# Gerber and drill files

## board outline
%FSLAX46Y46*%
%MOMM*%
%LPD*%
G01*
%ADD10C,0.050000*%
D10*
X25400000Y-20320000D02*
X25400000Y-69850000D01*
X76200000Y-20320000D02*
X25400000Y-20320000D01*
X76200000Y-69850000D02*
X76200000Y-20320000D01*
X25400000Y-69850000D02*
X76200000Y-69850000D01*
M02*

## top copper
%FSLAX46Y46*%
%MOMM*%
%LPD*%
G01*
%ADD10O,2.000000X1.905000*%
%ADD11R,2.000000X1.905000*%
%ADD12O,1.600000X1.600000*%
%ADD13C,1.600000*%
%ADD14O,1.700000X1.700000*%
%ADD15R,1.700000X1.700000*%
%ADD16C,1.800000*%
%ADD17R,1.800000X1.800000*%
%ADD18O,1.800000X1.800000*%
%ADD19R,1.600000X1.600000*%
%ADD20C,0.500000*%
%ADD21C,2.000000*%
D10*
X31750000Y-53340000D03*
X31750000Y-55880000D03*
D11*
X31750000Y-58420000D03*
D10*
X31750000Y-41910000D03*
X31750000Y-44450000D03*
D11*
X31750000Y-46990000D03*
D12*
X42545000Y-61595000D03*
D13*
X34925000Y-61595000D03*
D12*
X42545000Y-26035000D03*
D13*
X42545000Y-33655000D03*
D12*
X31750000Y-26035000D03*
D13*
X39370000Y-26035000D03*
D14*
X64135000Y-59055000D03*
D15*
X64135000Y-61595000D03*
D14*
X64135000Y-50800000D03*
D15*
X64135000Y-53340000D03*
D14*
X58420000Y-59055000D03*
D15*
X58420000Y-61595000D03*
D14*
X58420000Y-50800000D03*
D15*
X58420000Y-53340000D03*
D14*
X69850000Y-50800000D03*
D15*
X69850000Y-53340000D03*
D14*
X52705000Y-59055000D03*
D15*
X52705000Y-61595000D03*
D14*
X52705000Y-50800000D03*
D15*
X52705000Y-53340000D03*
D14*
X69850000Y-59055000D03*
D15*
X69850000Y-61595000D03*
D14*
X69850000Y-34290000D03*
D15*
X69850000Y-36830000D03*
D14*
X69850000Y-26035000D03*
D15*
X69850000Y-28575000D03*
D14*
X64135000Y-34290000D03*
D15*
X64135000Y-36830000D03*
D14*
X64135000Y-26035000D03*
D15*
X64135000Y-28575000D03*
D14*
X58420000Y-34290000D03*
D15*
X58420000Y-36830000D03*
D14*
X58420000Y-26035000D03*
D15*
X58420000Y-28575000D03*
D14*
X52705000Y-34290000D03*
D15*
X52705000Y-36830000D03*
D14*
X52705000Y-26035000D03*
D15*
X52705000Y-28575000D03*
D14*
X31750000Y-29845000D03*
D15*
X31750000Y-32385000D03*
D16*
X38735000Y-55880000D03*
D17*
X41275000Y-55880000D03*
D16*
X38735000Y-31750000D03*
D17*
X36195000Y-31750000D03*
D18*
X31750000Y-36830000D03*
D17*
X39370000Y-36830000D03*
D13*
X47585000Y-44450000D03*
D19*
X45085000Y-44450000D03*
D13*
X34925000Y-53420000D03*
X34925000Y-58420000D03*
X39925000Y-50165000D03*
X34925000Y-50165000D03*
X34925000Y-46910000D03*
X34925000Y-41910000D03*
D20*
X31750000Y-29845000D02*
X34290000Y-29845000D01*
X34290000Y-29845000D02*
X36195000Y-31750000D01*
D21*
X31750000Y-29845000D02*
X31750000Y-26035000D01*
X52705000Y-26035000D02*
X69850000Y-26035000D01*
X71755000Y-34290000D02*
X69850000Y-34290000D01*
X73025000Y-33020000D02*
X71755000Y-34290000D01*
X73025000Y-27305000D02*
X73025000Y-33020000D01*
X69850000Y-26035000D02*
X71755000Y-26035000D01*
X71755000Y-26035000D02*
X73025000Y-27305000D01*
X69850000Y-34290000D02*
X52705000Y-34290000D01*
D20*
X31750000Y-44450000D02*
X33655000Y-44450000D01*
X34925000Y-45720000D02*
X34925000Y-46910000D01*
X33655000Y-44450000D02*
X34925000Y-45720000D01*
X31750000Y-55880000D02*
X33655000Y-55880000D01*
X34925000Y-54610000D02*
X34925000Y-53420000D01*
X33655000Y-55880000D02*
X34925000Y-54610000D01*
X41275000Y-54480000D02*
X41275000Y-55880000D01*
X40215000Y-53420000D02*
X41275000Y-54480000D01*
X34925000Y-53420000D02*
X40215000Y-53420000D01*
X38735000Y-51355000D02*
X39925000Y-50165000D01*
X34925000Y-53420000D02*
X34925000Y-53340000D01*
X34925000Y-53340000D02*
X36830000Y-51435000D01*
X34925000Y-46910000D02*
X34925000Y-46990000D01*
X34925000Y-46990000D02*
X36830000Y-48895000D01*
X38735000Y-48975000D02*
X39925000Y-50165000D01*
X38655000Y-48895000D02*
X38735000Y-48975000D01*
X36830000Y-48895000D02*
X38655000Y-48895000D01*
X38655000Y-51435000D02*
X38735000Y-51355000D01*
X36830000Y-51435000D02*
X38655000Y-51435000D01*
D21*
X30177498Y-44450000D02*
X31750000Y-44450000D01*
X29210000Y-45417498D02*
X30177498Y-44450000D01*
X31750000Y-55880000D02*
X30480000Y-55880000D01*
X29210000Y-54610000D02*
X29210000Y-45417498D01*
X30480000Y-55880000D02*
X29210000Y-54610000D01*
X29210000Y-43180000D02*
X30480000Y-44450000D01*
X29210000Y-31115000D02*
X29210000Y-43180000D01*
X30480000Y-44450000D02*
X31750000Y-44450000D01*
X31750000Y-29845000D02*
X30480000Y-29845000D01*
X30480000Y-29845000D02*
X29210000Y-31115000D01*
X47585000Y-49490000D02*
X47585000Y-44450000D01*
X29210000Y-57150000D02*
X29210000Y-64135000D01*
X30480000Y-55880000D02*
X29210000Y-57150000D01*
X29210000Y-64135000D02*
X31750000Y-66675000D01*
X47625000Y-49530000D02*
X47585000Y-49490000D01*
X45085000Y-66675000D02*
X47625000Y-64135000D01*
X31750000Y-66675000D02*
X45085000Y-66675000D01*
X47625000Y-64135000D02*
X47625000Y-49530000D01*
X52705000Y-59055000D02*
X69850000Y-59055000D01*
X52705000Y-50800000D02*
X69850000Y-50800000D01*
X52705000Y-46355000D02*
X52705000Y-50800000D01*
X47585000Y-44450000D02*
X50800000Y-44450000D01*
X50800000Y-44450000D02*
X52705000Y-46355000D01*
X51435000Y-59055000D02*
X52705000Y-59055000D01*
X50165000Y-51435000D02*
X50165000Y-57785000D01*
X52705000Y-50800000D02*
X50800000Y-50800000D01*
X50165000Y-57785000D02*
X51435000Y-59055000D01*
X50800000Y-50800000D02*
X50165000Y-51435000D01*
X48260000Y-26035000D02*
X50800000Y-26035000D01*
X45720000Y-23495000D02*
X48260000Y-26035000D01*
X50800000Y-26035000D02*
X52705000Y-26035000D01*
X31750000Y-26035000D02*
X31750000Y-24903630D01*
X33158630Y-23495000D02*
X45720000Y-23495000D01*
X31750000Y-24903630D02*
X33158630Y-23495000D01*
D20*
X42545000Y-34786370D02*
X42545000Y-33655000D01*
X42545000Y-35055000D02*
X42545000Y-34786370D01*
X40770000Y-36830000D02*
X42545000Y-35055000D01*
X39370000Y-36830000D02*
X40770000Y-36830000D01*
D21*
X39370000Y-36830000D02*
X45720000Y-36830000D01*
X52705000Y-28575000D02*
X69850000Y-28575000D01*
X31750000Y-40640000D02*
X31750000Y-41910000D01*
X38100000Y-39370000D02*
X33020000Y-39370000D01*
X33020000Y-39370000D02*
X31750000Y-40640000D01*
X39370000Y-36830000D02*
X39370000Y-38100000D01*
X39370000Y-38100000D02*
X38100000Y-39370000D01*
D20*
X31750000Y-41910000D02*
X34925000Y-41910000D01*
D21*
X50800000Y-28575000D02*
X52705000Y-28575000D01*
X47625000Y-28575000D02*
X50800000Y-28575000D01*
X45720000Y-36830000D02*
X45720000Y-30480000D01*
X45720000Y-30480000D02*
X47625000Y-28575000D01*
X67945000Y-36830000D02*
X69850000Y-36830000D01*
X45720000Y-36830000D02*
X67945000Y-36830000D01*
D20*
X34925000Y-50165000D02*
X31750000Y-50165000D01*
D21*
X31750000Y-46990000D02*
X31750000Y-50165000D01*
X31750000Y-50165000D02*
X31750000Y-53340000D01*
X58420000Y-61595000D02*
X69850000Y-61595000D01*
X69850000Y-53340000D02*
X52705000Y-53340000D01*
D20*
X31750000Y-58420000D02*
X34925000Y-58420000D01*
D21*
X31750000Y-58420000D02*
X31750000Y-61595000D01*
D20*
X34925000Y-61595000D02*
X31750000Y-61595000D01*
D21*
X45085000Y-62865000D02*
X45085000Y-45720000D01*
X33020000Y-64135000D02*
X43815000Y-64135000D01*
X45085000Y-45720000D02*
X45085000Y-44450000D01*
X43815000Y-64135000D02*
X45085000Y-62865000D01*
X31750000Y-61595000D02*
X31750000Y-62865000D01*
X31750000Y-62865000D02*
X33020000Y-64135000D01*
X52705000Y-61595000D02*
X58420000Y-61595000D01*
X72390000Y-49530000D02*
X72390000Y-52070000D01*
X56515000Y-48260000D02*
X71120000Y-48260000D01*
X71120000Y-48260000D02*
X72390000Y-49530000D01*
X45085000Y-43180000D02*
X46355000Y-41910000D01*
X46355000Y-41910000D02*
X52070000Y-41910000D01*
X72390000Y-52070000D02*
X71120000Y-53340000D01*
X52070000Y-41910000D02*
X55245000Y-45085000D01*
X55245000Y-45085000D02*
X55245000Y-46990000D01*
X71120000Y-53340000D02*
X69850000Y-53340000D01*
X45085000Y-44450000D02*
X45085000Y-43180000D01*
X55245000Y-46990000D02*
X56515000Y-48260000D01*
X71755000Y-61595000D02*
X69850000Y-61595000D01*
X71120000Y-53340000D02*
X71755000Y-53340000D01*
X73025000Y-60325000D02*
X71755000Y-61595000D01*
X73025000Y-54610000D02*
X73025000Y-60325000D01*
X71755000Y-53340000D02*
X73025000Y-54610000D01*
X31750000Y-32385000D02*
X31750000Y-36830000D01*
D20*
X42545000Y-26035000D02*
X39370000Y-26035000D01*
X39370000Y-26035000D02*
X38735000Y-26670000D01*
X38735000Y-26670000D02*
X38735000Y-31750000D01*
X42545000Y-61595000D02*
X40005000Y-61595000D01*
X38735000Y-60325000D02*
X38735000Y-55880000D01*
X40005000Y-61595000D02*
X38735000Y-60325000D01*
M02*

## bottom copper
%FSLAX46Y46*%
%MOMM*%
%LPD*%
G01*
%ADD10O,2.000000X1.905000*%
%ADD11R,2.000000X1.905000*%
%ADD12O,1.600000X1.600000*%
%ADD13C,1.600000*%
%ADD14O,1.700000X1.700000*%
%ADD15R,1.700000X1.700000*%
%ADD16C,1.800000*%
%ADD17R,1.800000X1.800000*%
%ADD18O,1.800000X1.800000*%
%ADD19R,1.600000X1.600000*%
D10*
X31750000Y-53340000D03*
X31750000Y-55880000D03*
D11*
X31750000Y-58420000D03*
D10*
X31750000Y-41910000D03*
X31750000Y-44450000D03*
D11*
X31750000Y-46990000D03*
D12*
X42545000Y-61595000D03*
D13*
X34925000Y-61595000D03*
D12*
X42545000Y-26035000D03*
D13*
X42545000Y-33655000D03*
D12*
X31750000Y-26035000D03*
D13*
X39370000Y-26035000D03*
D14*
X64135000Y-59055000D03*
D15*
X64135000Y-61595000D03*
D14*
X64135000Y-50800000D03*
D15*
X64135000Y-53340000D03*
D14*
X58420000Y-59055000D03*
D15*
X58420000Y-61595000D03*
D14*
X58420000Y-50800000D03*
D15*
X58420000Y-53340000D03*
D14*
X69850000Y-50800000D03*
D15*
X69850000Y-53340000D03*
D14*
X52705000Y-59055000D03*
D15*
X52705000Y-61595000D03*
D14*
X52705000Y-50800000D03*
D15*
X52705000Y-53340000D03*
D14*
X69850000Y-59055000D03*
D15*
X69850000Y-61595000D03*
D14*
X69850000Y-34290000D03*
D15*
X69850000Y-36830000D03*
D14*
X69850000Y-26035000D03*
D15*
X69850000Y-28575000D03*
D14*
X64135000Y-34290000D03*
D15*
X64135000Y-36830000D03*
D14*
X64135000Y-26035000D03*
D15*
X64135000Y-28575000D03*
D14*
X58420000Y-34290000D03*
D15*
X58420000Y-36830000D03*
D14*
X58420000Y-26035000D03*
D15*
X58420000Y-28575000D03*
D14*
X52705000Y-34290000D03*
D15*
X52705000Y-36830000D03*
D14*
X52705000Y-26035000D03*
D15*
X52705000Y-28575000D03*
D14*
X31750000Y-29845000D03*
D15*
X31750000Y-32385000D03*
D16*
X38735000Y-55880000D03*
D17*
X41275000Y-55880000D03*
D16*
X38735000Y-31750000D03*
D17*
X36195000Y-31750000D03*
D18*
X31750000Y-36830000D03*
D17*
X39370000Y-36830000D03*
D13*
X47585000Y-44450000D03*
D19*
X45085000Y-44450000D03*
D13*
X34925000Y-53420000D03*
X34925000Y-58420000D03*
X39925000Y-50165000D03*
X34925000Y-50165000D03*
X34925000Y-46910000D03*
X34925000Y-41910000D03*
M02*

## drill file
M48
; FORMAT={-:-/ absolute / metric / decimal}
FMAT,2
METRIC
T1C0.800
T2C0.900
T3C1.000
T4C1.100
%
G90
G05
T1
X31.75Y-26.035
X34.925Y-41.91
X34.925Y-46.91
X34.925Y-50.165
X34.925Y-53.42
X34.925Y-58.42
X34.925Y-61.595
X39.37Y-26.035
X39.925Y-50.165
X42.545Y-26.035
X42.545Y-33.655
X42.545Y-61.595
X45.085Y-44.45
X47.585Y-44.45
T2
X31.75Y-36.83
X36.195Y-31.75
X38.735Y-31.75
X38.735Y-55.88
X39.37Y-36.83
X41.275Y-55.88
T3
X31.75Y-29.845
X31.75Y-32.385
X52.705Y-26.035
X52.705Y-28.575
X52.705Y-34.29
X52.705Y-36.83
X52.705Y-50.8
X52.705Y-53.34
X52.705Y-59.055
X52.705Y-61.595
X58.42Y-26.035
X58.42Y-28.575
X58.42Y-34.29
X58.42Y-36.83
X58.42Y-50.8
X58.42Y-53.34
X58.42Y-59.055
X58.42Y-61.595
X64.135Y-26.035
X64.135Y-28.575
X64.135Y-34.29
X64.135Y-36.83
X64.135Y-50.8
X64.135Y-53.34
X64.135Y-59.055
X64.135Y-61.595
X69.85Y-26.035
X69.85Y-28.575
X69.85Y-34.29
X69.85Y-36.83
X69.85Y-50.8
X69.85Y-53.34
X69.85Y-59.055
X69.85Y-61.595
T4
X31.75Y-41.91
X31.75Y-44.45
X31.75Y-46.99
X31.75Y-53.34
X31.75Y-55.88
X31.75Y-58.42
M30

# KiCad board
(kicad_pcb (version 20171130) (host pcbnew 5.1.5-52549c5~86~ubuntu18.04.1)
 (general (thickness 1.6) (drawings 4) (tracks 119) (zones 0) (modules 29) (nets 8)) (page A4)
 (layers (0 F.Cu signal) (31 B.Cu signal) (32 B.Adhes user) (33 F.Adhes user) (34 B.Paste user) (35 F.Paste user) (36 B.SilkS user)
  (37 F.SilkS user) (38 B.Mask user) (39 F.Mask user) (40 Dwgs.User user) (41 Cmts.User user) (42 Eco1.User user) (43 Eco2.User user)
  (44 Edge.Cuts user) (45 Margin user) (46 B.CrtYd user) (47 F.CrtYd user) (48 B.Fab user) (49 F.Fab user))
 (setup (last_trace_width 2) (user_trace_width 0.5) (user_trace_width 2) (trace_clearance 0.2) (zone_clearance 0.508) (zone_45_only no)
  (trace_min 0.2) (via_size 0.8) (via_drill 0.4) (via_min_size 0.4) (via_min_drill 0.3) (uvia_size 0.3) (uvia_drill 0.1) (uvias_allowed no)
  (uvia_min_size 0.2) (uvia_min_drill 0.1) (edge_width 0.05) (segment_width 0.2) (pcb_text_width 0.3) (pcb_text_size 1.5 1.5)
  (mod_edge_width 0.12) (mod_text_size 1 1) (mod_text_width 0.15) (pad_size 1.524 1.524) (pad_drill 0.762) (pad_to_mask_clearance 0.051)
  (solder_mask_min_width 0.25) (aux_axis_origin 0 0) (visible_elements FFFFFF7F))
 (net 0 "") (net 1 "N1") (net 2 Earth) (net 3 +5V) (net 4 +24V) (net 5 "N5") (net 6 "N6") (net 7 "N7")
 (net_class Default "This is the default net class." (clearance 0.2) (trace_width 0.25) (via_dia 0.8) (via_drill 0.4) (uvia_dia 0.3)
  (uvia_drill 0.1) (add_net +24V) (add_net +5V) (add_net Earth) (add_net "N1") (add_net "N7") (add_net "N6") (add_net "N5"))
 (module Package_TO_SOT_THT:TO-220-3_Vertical (layer F.Cu) (at 31.75 58.42 90)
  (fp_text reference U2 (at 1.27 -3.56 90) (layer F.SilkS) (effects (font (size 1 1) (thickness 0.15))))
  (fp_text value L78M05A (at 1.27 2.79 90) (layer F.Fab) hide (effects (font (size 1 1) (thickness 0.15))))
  (pad 3 thru_hole oval (at 5.08 0 90) (size 1.905 2) (drill 1.1) (layers *.Cu *.Mask) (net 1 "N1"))
  (pad 2 thru_hole oval (at 2.54 0 90) (size 1.905 2) (drill 1.1) (layers *.Cu *.Mask) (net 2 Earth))
  (pad 1 thru_hole rect (at 0 0 90) (size 1.905 2) (drill 1.1) (layers *.Cu *.Mask) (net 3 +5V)))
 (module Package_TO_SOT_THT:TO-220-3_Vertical (layer F.Cu) (at 31.75 46.99 90)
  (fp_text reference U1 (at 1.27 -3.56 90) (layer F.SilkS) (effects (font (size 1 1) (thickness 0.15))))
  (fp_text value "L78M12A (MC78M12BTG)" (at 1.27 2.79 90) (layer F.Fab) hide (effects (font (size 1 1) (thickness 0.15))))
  (pad 3 thru_hole oval (at 5.08 0 90) (size 1.905 2) (drill 1.1) (layers *.Cu *.Mask) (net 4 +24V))
  (pad 2 thru_hole oval (at 2.54 0 90) (size 1.905 2) (drill 1.1) (layers *.Cu *.Mask) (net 2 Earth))
  (pad 1 thru_hole rect (at 0 0 90) (size 1.905 2) (drill 1.1) (layers *.Cu *.Mask) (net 1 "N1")))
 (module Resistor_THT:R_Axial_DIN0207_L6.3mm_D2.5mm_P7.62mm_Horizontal (layer F.Cu) (at 34.925 61.595)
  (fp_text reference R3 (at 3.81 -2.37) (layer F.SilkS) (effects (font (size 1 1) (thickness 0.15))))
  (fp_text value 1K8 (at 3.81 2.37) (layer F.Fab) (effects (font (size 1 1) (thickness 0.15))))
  (pad 2 thru_hole oval (at 7.62 0) (size 1.6 1.6) (drill 0.8) (layers *.Cu *.Mask) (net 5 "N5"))
  (pad 1 thru_hole circle (at 0 0) (size 1.6 1.6) (drill 0.8) (layers *.Cu *.Mask) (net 3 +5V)))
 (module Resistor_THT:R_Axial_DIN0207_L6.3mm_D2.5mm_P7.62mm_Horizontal (layer F.Cu) (at 42.545 33.655 90)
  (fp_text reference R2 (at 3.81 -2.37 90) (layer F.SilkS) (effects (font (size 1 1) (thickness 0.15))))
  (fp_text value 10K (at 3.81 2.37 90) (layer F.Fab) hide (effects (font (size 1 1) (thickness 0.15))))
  (pad 2 thru_hole oval (at 7.62 0 90) (size 1.6 1.6) (drill 0.8) (layers *.Cu *.Mask) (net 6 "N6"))
  (pad 1 thru_hole circle (at 0 0 90) (size 1.6 1.6) (drill 0.8) (layers *.Cu *.Mask) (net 4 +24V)))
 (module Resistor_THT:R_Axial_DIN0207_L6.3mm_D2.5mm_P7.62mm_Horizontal (layer F.Cu) (at 39.37 26.035 180)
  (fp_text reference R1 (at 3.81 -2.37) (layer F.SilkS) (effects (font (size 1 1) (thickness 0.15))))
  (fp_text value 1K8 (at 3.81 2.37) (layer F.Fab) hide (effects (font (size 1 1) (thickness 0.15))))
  (pad 2 thru_hole oval (at 7.62 0 180) (size 1.6 1.6) (drill 0.8) (layers *.Cu *.Mask) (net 2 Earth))
  (pad 1 thru_hole circle (at 0 0 180) (size 1.6 1.6) (drill 0.8) (layers *.Cu *.Mask) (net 6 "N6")))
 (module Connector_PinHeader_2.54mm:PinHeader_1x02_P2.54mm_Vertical (layer F.Cu) (at 64.135 61.595 180)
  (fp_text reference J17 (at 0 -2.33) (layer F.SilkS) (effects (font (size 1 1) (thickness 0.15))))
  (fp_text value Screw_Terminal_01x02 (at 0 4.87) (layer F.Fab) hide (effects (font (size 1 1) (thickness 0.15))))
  (pad 2 thru_hole oval (at 0 2.54 180) (size 1.7 1.7) (drill 1) (layers *.Cu *.Mask) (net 2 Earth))
  (pad 1 thru_hole rect (at 0 0 180) (size 1.7 1.7) (drill 1) (layers *.Cu *.Mask) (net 3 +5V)))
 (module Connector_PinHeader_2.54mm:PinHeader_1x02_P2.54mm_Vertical (layer F.Cu) (at 64.135 53.34 180)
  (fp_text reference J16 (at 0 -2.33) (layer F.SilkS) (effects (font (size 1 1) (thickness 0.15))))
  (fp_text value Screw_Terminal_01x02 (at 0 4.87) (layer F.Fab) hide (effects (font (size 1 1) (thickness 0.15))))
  (pad 2 thru_hole oval (at 0 2.54 180) (size 1.7 1.7) (drill 1) (layers *.Cu *.Mask) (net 2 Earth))
  (pad 1 thru_hole rect (at 0 0 180) (size 1.7 1.7) (drill 1) (layers *.Cu *.Mask) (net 3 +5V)))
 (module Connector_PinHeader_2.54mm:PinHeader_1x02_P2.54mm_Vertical (layer F.Cu) (at 58.42 61.595 180)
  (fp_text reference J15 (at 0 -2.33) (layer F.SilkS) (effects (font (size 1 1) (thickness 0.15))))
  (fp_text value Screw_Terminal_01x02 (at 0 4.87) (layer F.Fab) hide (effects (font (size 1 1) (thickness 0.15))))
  (pad 2 thru_hole oval (at 0 2.54 180) (size 1.7 1.7) (drill 1) (layers *.Cu *.Mask) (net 2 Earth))
  (pad 1 thru_hole rect (at 0 0 180) (size 1.7 1.7) (drill 1) (layers *.Cu *.Mask) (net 3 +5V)))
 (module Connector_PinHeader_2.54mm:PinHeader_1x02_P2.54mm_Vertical (layer F.Cu) (at 58.42 53.34 180)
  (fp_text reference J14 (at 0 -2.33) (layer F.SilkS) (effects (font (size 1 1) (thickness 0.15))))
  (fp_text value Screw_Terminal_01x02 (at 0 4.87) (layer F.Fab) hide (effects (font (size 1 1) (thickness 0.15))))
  (pad 2 thru_hole oval (at 0 2.54 180) (size 1.7 1.7) (drill 1) (layers *.Cu *.Mask) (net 2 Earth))
  (pad 1 thru_hole rect (at 0 0 180) (size 1.7 1.7) (drill 1) (layers *.Cu *.Mask) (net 3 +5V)))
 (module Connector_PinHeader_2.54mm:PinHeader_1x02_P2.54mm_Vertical (layer F.Cu) (at 69.85 53.34 180)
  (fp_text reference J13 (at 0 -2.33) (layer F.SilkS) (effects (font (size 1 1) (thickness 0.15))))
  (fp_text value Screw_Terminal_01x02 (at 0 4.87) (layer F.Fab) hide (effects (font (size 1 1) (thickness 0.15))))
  (pad 2 thru_hole oval (at 0 2.54 180) (size 1.7 1.7) (drill 1) (layers *.Cu *.Mask) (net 2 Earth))
  (pad 1 thru_hole rect (at 0 0 180) (size 1.7 1.7) (drill 1) (layers *.Cu *.Mask) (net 3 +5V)))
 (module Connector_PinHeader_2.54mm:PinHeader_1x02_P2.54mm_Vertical (layer F.Cu) (at 52.705 61.595 180)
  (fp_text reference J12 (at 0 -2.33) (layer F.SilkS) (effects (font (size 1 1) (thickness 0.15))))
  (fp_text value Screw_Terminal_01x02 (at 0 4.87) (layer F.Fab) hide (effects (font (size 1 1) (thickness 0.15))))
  (pad 2 thru_hole oval (at 0 2.54 180) (size 1.7 1.7) (drill 1) (layers *.Cu *.Mask) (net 2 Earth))
  (pad 1 thru_hole rect (at 0 0 180) (size 1.7 1.7) (drill 1) (layers *.Cu *.Mask) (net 3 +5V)))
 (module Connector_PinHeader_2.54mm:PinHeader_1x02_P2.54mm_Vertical (layer F.Cu) (at 52.705 53.34 180)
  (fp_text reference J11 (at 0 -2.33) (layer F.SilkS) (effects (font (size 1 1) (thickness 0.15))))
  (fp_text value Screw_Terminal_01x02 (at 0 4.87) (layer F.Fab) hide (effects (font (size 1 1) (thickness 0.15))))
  (pad 2 thru_hole oval (at 0 2.54 180) (size 1.7 1.7) (drill 1) (layers *.Cu *.Mask) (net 2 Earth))
  (pad 1 thru_hole rect (at 0 0 180) (size 1.7 1.7) (drill 1) (layers *.Cu *.Mask) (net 3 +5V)))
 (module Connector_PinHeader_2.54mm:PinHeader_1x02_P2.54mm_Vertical (layer F.Cu) (at 69.85 61.595 180)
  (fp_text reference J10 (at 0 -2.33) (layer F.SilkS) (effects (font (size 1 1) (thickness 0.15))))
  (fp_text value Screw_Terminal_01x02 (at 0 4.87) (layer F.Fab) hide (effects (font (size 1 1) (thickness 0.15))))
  (pad 2 thru_hole oval (at 0 2.54 180) (size 1.7 1.7) (drill 1) (layers *.Cu *.Mask) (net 2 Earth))
  (pad 1 thru_hole rect (at 0 0 180) (size 1.7 1.7) (drill 1) (layers *.Cu *.Mask) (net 3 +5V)))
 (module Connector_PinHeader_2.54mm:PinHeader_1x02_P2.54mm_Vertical (layer F.Cu) (at 69.85 36.83 180)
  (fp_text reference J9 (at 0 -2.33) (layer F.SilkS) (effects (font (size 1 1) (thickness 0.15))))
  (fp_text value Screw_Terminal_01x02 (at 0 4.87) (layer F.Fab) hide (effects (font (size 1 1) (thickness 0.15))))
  (pad 2 thru_hole oval (at 0 2.54 180) (size 1.7 1.7) (drill 1) (layers *.Cu *.Mask) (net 2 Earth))
  (pad 1 thru_hole rect (at 0 0 180) (size 1.7 1.7) (drill 1) (layers *.Cu *.Mask) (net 4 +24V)))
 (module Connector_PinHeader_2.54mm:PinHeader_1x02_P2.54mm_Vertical (layer F.Cu) (at 69.85 28.575 180)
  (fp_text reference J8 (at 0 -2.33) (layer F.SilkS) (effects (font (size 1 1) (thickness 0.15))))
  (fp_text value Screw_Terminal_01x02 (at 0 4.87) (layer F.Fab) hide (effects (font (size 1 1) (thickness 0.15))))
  (pad 2 thru_hole oval (at 0 2.54 180) (size 1.7 1.7) (drill 1) (layers *.Cu *.Mask) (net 2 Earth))
  (pad 1 thru_hole rect (at 0 0 180) (size 1.7 1.7) (drill 1) (layers *.Cu *.Mask) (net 4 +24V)))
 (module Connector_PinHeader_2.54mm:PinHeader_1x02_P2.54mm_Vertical (layer F.Cu) (at 64.135 36.83 180)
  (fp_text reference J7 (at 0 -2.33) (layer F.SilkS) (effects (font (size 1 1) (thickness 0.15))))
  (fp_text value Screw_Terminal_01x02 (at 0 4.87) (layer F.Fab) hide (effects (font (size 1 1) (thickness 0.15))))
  (pad 2 thru_hole oval (at 0 2.54 180) (size 1.7 1.7) (drill 1) (layers *.Cu *.Mask) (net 2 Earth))
  (pad 1 thru_hole rect (at 0 0 180) (size 1.7 1.7) (drill 1) (layers *.Cu *.Mask) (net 4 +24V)))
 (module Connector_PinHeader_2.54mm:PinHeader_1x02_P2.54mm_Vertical (layer F.Cu) (at 64.135 28.575 180)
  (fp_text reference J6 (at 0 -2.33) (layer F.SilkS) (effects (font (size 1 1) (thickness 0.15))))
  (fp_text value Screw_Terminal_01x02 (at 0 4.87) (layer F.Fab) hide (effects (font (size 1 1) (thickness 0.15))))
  (pad 2 thru_hole oval (at 0 2.54 180) (size 1.7 1.7) (drill 1) (layers *.Cu *.Mask) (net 2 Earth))
  (pad 1 thru_hole rect (at 0 0 180) (size 1.7 1.7) (drill 1) (layers *.Cu *.Mask) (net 4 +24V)))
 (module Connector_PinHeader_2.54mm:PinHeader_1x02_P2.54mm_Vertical (layer F.Cu) (at 58.42 36.83 180)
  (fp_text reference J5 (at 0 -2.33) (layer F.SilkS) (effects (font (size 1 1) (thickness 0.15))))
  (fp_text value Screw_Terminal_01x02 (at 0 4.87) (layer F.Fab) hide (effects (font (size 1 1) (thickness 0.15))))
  (pad 2 thru_hole oval (at 0 2.54 180) (size 1.7 1.7) (drill 1) (layers *.Cu *.Mask) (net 2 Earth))
  (pad 1 thru_hole rect (at 0 0 180) (size 1.7 1.7) (drill 1) (layers *.Cu *.Mask) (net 4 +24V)))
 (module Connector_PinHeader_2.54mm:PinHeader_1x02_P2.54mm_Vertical (layer F.Cu) (at 58.42 28.575 180)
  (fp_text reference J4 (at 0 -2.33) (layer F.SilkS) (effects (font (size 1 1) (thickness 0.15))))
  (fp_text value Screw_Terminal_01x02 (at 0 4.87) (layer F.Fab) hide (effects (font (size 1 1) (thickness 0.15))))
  (pad 2 thru_hole oval (at 0 2.54 180) (size 1.7 1.7) (drill 1) (layers *.Cu *.Mask) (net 2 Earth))
  (pad 1 thru_hole rect (at 0 0 180) (size 1.7 1.7) (drill 1) (layers *.Cu *.Mask) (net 4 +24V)))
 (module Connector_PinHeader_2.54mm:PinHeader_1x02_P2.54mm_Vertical (layer F.Cu) (at 52.705 36.83 180)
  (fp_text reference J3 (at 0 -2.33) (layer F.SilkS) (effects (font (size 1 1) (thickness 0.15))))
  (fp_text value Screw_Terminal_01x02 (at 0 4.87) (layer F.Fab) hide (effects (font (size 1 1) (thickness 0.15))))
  (pad 2 thru_hole oval (at 0 2.54 180) (size 1.7 1.7) (drill 1) (layers *.Cu *.Mask) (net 2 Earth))
  (pad 1 thru_hole rect (at 0 0 180) (size 1.7 1.7) (drill 1) (layers *.Cu *.Mask) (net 4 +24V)))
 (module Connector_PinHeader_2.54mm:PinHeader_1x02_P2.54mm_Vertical (layer F.Cu) (at 52.705 28.575 180)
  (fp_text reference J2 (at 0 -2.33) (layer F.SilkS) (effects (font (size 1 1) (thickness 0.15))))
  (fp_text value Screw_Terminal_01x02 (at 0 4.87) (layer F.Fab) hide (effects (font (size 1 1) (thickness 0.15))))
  (pad 2 thru_hole oval (at 0 2.54 180) (size 1.7 1.7) (drill 1) (layers *.Cu *.Mask) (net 2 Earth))
  (pad 1 thru_hole rect (at 0 0 180) (size 1.7 1.7) (drill 1) (layers *.Cu *.Mask) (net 4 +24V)))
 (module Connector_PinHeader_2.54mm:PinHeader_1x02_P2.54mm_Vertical (layer F.Cu) (at 31.75 32.385 180)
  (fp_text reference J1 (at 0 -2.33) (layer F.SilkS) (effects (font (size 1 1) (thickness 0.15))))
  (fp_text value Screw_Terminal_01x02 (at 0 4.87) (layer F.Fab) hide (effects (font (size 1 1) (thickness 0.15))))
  (pad 2 thru_hole oval (at 0 2.54 180) (size 1.7 1.7) (drill 1) (layers *.Cu *.Mask) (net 2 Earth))
  (pad 1 thru_hole rect (at 0 0 180) (size 1.7 1.7) (drill 1) (layers *.Cu *.Mask) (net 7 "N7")))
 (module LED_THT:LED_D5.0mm (layer F.Cu) (at 41.275 55.88 180)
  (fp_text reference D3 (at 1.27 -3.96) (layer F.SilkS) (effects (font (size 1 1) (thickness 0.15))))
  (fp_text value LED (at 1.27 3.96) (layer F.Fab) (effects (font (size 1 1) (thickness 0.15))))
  (pad 2 thru_hole circle (at 2.54 0 180) (size 1.8 1.8) (drill 0.9) (layers *.Cu *.Mask) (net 5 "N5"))
  (pad 1 thru_hole rect (at 0 0 180) (size 1.8 1.8) (drill 0.9) (layers *.Cu *.Mask) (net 2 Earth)))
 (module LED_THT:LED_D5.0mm (layer F.Cu) (at 36.195 31.75)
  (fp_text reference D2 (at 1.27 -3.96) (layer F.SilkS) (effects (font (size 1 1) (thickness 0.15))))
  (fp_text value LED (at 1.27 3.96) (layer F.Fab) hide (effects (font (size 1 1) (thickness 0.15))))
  (pad 2 thru_hole circle (at 2.54 0) (size 1.8 1.8) (drill 0.9) (layers *.Cu *.Mask) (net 6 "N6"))
  (pad 1 thru_hole rect (at 0 0) (size 1.8 1.8) (drill 0.9) (layers *.Cu *.Mask) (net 2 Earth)))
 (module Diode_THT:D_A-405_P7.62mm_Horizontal (layer F.Cu) (at 39.37 36.83 180)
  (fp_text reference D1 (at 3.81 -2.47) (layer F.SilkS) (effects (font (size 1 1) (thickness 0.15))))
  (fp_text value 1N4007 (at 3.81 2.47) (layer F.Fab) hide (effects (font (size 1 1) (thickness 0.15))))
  (pad 2 thru_hole oval (at 7.62 0 180) (size 1.8 1.8) (drill 0.9) (layers *.Cu *.Mask) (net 7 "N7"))
  (pad 1 thru_hole rect (at 0 0 180) (size 1.8 1.8) (drill 0.9) (layers *.Cu *.Mask) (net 4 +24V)))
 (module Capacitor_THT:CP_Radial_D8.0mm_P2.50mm (layer F.Cu) (at 45.085 44.45)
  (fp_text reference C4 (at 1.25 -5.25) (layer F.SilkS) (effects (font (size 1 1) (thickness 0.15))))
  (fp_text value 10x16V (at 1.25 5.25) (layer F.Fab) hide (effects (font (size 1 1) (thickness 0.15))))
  (pad 2 thru_hole circle (at 2.5 0) (size 1.6 1.6) (drill 0.8) (layers *.Cu *.Mask) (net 2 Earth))
  (pad 1 thru_hole rect (at 0 0) (size 1.6 1.6) (drill 0.8) (layers *.Cu *.Mask) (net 3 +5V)))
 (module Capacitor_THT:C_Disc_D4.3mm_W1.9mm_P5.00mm (layer F.Cu) (at 34.925 58.42 90)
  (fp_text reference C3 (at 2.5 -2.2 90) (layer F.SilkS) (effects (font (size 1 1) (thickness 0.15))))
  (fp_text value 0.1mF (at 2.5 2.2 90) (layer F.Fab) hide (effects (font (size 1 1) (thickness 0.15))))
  (pad 2 thru_hole circle (at 5 0 90) (size 1.6 1.6) (drill 0.8) (layers *.Cu *.Mask) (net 2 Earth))
  (pad 1 thru_hole circle (at 0 0 90) (size 1.6 1.6) (drill 0.8) (layers *.Cu *.Mask) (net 3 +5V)))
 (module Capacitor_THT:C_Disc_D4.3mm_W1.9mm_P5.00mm (layer F.Cu) (at 34.925 50.165)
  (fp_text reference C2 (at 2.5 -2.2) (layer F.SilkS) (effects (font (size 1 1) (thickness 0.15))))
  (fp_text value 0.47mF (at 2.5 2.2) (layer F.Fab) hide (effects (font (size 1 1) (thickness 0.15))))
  (pad 2 thru_hole circle (at 5 0) (size 1.6 1.6) (drill 0.8) (layers *.Cu *.Mask) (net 2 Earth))
  (pad 1 thru_hole circle (at 0 0) (size 1.6 1.6) (drill 0.8) (layers *.Cu *.Mask) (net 1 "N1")))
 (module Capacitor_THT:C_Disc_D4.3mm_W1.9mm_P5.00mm (layer F.Cu) (at 34.925 41.91 270)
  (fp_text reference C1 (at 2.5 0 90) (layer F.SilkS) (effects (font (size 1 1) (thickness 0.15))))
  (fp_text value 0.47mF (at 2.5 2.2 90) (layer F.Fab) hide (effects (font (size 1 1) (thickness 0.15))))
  (pad 2 thru_hole circle (at 5 0 270) (size 1.6 1.6) (drill 0.8) (layers *.Cu *.Mask) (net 2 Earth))
  (pad 1 thru_hole circle (at 0 0 270) (size 1.6 1.6) (drill 0.8) (layers *.Cu *.Mask) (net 4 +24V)))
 (gr_line (start 25.4 20.32) (end 25.4 69.85) (layer Edge.Cuts) (width 0.05))
 (gr_line (start 76.2 20.32) (end 25.4 20.32) (layer Edge.Cuts) (width 0.05))
 (gr_line (start 76.2 69.85) (end 76.2 20.32) (layer Edge.Cuts) (width 0.05))
 (gr_line (start 25.4 69.85) (end 76.2 69.85) (layer Edge.Cuts) (width 0.05))
 (segment (start 31.75 29.845) (end 34.29 29.845) (width 0.5) (layer F.Cu) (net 2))
 (segment (start 34.29 29.845) (end 36.195 31.75) (width 0.5) (layer F.Cu) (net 2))
 (segment (start 31.75 29.845) (end 31.75 26.035) (width 2) (layer F.Cu) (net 2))
 (segment (start 52.705 26.035) (end 69.85 26.035) (width 2) (layer F.Cu) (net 2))
 (segment (start 71.755 34.29) (end 69.85 34.29) (width 2) (layer F.Cu) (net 2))
 (segment (start 73.025 33.02) (end 71.755 34.29) (width 2) (layer F.Cu) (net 2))
 (segment (start 73.025 27.305) (end 73.025 33.02) (width 2) (layer F.Cu) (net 2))
 (segment (start 69.85 26.035) (end 71.755 26.035) (width 2) (layer F.Cu) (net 2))
 (segment (start 71.755 26.035) (end 73.025 27.305) (width 2) (layer F.Cu) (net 2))
 (segment (start 69.85 34.29) (end 52.705 34.29) (width 2) (layer F.Cu) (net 2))
 (segment (start 31.75 44.45) (end 33.655 44.45) (width 0.5) (layer F.Cu) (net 2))
 (segment (start 34.925 45.72) (end 34.925 46.91) (width 0.5) (layer F.Cu) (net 2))
 (segment (start 33.655 44.45) (end 34.925 45.72) (width 0.5) (layer F.Cu) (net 2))
 (segment (start 31.75 55.88) (end 33.655 55.88) (width 0.5) (layer F.Cu) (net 2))
 (segment (start 34.925 54.61) (end 34.925 53.42) (width 0.5) (layer F.Cu) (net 2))
 (segment (start 33.655 55.88) (end 34.925 54.61) (width 0.5) (layer F.Cu) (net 2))
 (segment (start 41.275 54.48) (end 41.275 55.88) (width 0.5) (layer F.Cu) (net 2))
 (segment (start 40.215 53.42) (end 41.275 54.48) (width 0.5) (layer F.Cu) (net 2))
 (segment (start 34.925 53.42) (end 40.215 53.42) (width 0.5) (layer F.Cu) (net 2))
 (segment (start 38.735 51.355) (end 39.925 50.165) (width 0.5) (layer F.Cu) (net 2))
 (segment (start 34.925 53.42) (end 34.925 53.34) (width 0.5) (layer F.Cu) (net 2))
 (segment (start 34.925 53.34) (end 36.83 51.435) (width 0.5) (layer F.Cu) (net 2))
 (segment (start 34.925 46.91) (end 34.925 46.99) (width 0.5) (layer F.Cu) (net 2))
 (segment (start 34.925 46.99) (end 36.83 48.895) (width 0.5) (layer F.Cu) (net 2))
 (segment (start 38.735 48.975) (end 39.925 50.165) (width 0.5) (layer F.Cu) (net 2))
 (segment (start 38.655 48.895) (end 38.735 48.975) (width 0.5) (layer F.Cu) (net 2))
 (segment (start 36.83 48.895) (end 38.655 48.895) (width 0.5) (layer F.Cu) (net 2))
 (segment (start 38.655 51.435) (end 38.735 51.355) (width 0.5) (layer F.Cu) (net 2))
 (segment (start 36.83 51.435) (end 38.655 51.435) (width 0.5) (layer F.Cu) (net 2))
 (segment (start 30.177498 44.45) (end 31.75 44.45) (width 2) (layer F.Cu) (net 2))
 (segment (start 29.21 45.417498) (end 30.177498 44.45) (width 2) (layer F.Cu) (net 2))
 (segment (start 31.75 55.88) (end 30.48 55.88) (width 2) (layer F.Cu) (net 2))
 (segment (start 29.21 54.61) (end 29.21 45.417498) (width 2) (layer F.Cu) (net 2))
 (segment (start 30.48 55.88) (end 29.21 54.61) (width 2) (layer F.Cu) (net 2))
 (segment (start 29.21 43.18) (end 30.48 44.45) (width 2) (layer F.Cu) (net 2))
 (segment (start 29.21 31.115) (end 29.21 43.18) (width 2) (layer F.Cu) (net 2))
 (segment (start 30.48 44.45) (end 31.75 44.45) (width 2) (layer F.Cu) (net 2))
 (segment (start 31.75 29.845) (end 30.48 29.845) (width 2) (layer F.Cu) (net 2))
 (segment (start 30.48 29.845) (end 29.21 31.115) (width 2) (layer F.Cu) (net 2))
 (segment (start 47.585 49.49) (end 47.585 44.45) (width 2) (layer F.Cu) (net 2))
 (segment (start 29.21 57.15) (end 29.21 64.135) (width 2) (layer F.Cu) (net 2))
 (segment (start 30.48 55.88) (end 29.21 57.15) (width 2) (layer F.Cu) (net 2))
 (segment (start 29.21 64.135) (end 31.75 66.675) (width 2) (layer F.Cu) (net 2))
 (segment (start 47.625 49.53) (end 47.585 49.49) (width 2) (layer F.Cu) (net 2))
 (segment (start 45.085 66.675) (end 47.625 64.135) (width 2) (layer F.Cu) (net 2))
 (segment (start 31.75 66.675) (end 45.085 66.675) (width 2) (layer F.Cu) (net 2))
 (segment (start 47.625 64.135) (end 47.625 49.53) (width 2) (layer F.Cu) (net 2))
 (segment (start 52.705 59.055) (end 69.85 59.055) (width 2) (layer F.Cu) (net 2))
 (segment (start 52.705 50.8) (end 69.85 50.8) (width 2) (layer F.Cu) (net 2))
 (segment (start 52.705 46.355) (end 52.705 50.8) (width 2) (layer F.Cu) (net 2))
 (segment (start 47.585 44.45) (end 50.8 44.45) (width 2) (layer F.Cu) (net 2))
 (segment (start 50.8 44.45) (end 52.705 46.355) (width 2) (layer F.Cu) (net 2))
 (segment (start 51.435 59.055) (end 52.705 59.055) (width 2) (layer F.Cu) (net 2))
 (segment (start 50.165 51.435) (end 50.165 57.785) (width 2) (layer F.Cu) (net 2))
 (segment (start 52.705 50.8) (end 50.8 50.8) (width 2) (layer F.Cu) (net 2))
 (segment (start 50.165 57.785) (end 51.435 59.055) (width 2) (layer F.Cu) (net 2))
 (segment (start 50.8 50.8) (end 50.165 51.435) (width 2) (layer F.Cu) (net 2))
 (segment (start 48.26 26.035) (end 50.8 26.035) (width 2) (layer F.Cu) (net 2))
 (segment (start 45.72 23.495) (end 48.26 26.035) (width 2) (layer F.Cu) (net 2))
 (segment (start 50.8 26.035) (end 52.705 26.035) (width 2) (layer F.Cu) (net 2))
 (segment (start 31.75 26.035) (end 31.75 24.90363) (width 2) (layer F.Cu) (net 2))
 (segment (start 33.15863 23.495) (end 45.72 23.495) (width 2) (layer F.Cu) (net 2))
 (segment (start 31.75 24.90363) (end 33.15863 23.495) (width 2) (layer F.Cu) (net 2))
 (segment (start 42.545 34.78637) (end 42.545 33.655) (width 0.5) (layer F.Cu) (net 4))
 (segment (start 42.545 35.055) (end 42.545 34.78637) (width 0.5) (layer F.Cu) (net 4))
 (segment (start 40.77 36.83) (end 42.545 35.055) (width 0.5) (layer F.Cu) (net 4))
 (segment (start 39.37 36.83) (end 40.77 36.83) (width 0.5) (layer F.Cu) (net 4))
 (segment (start 39.37 36.83) (end 45.72 36.83) (width 2) (layer F.Cu) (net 4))
 (segment (start 52.705 28.575) (end 69.85 28.575) (width 2) (layer F.Cu) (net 4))
 (segment (start 31.75 40.64) (end 31.75 41.91) (width 2) (layer F.Cu) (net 4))
 (segment (start 38.1 39.37) (end 33.02 39.37) (width 2) (layer F.Cu) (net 4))
 (segment (start 33.02 39.37) (end 31.75 40.64) (width 2) (layer F.Cu) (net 4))
 (segment (start 39.37 36.83) (end 39.37 38.1) (width 2) (layer F.Cu) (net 4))
 (segment (start 39.37 38.1) (end 38.1 39.37) (width 2) (layer F.Cu) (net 4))
 (segment (start 31.75 41.91) (end 34.925 41.91) (width 0.5) (layer F.Cu) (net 4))
 (segment (start 50.8 28.575) (end 52.705 28.575) (width 2) (layer F.Cu) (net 4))
 (segment (start 47.625 28.575) (end 50.8 28.575) (width 2) (layer F.Cu) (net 4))
 (segment (start 45.72 36.83) (end 45.72 30.48) (width 2) (layer F.Cu) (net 4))
 (segment (start 45.72 30.48) (end 47.625 28.575) (width 2) (layer F.Cu) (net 4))
 (segment (start 67.945 36.83) (end 69.85 36.83) (width 2) (layer F.Cu) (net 4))
 (segment (start 45.72 36.83) (end 67.945 36.83) (width 2) (layer F.Cu) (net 4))
 (segment (start 34.925 50.165) (end 31.75 50.165) (width 0.5) (layer F.Cu) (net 1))
 (segment (start 31.75 46.99) (end 31.75 50.165) (width 2) (layer F.Cu) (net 1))
 (segment (start 31.75 50.165) (end 31.75 53.34) (width 2) (layer F.Cu) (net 1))
 (segment (start 58.42 61.595) (end 69.85 61.595) (width 2) (layer F.Cu) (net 3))
 (segment (start 69.85 53.34) (end 52.705 53.34) (width 2) (layer F.Cu) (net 3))
 (segment (start 31.75 58.42) (end 34.925 58.42) (width 0.5) (layer F.Cu) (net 3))
 (segment (start 31.75 58.42) (end 31.75 61.595) (width 2) (layer F.Cu) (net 3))
 (segment (start 34.925 61.595) (end 31.75 61.595) (width 0.5) (layer F.Cu) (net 3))
 (segment (start 45.085 62.865) (end 45.085 45.72) (width 2) (layer F.Cu) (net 3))
 (segment (start 33.02 64.135) (end 43.815 64.135) (width 2) (layer F.Cu) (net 3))
 (segment (start 45.085 45.72) (end 45.085 44.45) (width 2) (layer F.Cu) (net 3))
 (segment (start 43.815 64.135) (end 45.085 62.865) (width 2) (layer F.Cu) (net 3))
 (segment (start 31.75 61.595) (end 31.75 62.865) (width 2) (layer F.Cu) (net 3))
 (segment (start 31.75 62.865) (end 33.02 64.135) (width 2) (layer F.Cu) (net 3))
 (segment (start 52.705 61.595) (end 58.42 61.595) (width 2) (layer F.Cu) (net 3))
 (segment (start 72.39 49.53) (end 72.39 52.07) (width 2) (layer F.Cu) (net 3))
 (segment (start 56.515 48.26) (end 71.12 48.26) (width 2) (layer F.Cu) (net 3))
 (segment (start 71.12 48.26) (end 72.39 49.53) (width 2) (layer F.Cu) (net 3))
 (segment (start 45.085 43.18) (end 46.355 41.91) (width 2) (layer F.Cu) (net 3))
 (segment (start 46.355 41.91) (end 52.07 41.91) (width 2) (layer F.Cu) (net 3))
 (segment (start 72.39 52.07) (end 71.12 53.34) (width 2) (layer F.Cu) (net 3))
 (segment (start 52.07 41.91) (end 55.245 45.085) (width 2) (layer F.Cu) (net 3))
 (segment (start 55.245 45.085) (end 55.245 46.99) (width 2) (layer F.Cu) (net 3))
 (segment (start 71.12 53.34) (end 69.85 53.34) (width 2) (layer F.Cu) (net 3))
 (segment (start 45.085 44.45) (end 45.085 43.18) (width 2) (layer F.Cu) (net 3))
 (segment (start 55.245 46.99) (end 56.515 48.26) (width 2) (layer F.Cu) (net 3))
 (segment (start 71.755 61.595) (end 69.85 61.595) (width 2) (layer F.Cu) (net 3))
 (segment (start 71.12 53.34) (end 71.755 53.34) (width 2) (layer F.Cu) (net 3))
 (segment (start 73.025 60.325) (end 71.755 61.595) (width 2) (layer F.Cu) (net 3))
 (segment (start 73.025 54.61) (end 73.025 60.325) (width 2) (layer F.Cu) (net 3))
 (segment (start 71.755 53.34) (end 73.025 54.61) (width 2) (layer F.Cu) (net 3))
 (segment (start 31.75 32.385) (end 31.75 36.83) (width 2) (layer F.Cu) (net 7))
 (segment (start 42.545 26.035) (end 39.37 26.035) (width 0.5) (layer F.Cu) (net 6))
 (segment (start 39.37 26.035) (end 38.735 26.67) (width 0.5) (layer F.Cu) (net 6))
 (segment (start 38.735 26.67) (end 38.735 31.75) (width 0.5) (layer F.Cu) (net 6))
 (segment (start 42.545 61.595) (end 40.005 61.595) (width 0.5) (layer F.Cu) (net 5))
 (segment (start 38.735 60.325) (end 38.735 55.88) (width 0.5) (layer F.Cu) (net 5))
 (segment (start 40.005 61.595) (end 38.735 60.325) (width 0.5) (layer F.Cu) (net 5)))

